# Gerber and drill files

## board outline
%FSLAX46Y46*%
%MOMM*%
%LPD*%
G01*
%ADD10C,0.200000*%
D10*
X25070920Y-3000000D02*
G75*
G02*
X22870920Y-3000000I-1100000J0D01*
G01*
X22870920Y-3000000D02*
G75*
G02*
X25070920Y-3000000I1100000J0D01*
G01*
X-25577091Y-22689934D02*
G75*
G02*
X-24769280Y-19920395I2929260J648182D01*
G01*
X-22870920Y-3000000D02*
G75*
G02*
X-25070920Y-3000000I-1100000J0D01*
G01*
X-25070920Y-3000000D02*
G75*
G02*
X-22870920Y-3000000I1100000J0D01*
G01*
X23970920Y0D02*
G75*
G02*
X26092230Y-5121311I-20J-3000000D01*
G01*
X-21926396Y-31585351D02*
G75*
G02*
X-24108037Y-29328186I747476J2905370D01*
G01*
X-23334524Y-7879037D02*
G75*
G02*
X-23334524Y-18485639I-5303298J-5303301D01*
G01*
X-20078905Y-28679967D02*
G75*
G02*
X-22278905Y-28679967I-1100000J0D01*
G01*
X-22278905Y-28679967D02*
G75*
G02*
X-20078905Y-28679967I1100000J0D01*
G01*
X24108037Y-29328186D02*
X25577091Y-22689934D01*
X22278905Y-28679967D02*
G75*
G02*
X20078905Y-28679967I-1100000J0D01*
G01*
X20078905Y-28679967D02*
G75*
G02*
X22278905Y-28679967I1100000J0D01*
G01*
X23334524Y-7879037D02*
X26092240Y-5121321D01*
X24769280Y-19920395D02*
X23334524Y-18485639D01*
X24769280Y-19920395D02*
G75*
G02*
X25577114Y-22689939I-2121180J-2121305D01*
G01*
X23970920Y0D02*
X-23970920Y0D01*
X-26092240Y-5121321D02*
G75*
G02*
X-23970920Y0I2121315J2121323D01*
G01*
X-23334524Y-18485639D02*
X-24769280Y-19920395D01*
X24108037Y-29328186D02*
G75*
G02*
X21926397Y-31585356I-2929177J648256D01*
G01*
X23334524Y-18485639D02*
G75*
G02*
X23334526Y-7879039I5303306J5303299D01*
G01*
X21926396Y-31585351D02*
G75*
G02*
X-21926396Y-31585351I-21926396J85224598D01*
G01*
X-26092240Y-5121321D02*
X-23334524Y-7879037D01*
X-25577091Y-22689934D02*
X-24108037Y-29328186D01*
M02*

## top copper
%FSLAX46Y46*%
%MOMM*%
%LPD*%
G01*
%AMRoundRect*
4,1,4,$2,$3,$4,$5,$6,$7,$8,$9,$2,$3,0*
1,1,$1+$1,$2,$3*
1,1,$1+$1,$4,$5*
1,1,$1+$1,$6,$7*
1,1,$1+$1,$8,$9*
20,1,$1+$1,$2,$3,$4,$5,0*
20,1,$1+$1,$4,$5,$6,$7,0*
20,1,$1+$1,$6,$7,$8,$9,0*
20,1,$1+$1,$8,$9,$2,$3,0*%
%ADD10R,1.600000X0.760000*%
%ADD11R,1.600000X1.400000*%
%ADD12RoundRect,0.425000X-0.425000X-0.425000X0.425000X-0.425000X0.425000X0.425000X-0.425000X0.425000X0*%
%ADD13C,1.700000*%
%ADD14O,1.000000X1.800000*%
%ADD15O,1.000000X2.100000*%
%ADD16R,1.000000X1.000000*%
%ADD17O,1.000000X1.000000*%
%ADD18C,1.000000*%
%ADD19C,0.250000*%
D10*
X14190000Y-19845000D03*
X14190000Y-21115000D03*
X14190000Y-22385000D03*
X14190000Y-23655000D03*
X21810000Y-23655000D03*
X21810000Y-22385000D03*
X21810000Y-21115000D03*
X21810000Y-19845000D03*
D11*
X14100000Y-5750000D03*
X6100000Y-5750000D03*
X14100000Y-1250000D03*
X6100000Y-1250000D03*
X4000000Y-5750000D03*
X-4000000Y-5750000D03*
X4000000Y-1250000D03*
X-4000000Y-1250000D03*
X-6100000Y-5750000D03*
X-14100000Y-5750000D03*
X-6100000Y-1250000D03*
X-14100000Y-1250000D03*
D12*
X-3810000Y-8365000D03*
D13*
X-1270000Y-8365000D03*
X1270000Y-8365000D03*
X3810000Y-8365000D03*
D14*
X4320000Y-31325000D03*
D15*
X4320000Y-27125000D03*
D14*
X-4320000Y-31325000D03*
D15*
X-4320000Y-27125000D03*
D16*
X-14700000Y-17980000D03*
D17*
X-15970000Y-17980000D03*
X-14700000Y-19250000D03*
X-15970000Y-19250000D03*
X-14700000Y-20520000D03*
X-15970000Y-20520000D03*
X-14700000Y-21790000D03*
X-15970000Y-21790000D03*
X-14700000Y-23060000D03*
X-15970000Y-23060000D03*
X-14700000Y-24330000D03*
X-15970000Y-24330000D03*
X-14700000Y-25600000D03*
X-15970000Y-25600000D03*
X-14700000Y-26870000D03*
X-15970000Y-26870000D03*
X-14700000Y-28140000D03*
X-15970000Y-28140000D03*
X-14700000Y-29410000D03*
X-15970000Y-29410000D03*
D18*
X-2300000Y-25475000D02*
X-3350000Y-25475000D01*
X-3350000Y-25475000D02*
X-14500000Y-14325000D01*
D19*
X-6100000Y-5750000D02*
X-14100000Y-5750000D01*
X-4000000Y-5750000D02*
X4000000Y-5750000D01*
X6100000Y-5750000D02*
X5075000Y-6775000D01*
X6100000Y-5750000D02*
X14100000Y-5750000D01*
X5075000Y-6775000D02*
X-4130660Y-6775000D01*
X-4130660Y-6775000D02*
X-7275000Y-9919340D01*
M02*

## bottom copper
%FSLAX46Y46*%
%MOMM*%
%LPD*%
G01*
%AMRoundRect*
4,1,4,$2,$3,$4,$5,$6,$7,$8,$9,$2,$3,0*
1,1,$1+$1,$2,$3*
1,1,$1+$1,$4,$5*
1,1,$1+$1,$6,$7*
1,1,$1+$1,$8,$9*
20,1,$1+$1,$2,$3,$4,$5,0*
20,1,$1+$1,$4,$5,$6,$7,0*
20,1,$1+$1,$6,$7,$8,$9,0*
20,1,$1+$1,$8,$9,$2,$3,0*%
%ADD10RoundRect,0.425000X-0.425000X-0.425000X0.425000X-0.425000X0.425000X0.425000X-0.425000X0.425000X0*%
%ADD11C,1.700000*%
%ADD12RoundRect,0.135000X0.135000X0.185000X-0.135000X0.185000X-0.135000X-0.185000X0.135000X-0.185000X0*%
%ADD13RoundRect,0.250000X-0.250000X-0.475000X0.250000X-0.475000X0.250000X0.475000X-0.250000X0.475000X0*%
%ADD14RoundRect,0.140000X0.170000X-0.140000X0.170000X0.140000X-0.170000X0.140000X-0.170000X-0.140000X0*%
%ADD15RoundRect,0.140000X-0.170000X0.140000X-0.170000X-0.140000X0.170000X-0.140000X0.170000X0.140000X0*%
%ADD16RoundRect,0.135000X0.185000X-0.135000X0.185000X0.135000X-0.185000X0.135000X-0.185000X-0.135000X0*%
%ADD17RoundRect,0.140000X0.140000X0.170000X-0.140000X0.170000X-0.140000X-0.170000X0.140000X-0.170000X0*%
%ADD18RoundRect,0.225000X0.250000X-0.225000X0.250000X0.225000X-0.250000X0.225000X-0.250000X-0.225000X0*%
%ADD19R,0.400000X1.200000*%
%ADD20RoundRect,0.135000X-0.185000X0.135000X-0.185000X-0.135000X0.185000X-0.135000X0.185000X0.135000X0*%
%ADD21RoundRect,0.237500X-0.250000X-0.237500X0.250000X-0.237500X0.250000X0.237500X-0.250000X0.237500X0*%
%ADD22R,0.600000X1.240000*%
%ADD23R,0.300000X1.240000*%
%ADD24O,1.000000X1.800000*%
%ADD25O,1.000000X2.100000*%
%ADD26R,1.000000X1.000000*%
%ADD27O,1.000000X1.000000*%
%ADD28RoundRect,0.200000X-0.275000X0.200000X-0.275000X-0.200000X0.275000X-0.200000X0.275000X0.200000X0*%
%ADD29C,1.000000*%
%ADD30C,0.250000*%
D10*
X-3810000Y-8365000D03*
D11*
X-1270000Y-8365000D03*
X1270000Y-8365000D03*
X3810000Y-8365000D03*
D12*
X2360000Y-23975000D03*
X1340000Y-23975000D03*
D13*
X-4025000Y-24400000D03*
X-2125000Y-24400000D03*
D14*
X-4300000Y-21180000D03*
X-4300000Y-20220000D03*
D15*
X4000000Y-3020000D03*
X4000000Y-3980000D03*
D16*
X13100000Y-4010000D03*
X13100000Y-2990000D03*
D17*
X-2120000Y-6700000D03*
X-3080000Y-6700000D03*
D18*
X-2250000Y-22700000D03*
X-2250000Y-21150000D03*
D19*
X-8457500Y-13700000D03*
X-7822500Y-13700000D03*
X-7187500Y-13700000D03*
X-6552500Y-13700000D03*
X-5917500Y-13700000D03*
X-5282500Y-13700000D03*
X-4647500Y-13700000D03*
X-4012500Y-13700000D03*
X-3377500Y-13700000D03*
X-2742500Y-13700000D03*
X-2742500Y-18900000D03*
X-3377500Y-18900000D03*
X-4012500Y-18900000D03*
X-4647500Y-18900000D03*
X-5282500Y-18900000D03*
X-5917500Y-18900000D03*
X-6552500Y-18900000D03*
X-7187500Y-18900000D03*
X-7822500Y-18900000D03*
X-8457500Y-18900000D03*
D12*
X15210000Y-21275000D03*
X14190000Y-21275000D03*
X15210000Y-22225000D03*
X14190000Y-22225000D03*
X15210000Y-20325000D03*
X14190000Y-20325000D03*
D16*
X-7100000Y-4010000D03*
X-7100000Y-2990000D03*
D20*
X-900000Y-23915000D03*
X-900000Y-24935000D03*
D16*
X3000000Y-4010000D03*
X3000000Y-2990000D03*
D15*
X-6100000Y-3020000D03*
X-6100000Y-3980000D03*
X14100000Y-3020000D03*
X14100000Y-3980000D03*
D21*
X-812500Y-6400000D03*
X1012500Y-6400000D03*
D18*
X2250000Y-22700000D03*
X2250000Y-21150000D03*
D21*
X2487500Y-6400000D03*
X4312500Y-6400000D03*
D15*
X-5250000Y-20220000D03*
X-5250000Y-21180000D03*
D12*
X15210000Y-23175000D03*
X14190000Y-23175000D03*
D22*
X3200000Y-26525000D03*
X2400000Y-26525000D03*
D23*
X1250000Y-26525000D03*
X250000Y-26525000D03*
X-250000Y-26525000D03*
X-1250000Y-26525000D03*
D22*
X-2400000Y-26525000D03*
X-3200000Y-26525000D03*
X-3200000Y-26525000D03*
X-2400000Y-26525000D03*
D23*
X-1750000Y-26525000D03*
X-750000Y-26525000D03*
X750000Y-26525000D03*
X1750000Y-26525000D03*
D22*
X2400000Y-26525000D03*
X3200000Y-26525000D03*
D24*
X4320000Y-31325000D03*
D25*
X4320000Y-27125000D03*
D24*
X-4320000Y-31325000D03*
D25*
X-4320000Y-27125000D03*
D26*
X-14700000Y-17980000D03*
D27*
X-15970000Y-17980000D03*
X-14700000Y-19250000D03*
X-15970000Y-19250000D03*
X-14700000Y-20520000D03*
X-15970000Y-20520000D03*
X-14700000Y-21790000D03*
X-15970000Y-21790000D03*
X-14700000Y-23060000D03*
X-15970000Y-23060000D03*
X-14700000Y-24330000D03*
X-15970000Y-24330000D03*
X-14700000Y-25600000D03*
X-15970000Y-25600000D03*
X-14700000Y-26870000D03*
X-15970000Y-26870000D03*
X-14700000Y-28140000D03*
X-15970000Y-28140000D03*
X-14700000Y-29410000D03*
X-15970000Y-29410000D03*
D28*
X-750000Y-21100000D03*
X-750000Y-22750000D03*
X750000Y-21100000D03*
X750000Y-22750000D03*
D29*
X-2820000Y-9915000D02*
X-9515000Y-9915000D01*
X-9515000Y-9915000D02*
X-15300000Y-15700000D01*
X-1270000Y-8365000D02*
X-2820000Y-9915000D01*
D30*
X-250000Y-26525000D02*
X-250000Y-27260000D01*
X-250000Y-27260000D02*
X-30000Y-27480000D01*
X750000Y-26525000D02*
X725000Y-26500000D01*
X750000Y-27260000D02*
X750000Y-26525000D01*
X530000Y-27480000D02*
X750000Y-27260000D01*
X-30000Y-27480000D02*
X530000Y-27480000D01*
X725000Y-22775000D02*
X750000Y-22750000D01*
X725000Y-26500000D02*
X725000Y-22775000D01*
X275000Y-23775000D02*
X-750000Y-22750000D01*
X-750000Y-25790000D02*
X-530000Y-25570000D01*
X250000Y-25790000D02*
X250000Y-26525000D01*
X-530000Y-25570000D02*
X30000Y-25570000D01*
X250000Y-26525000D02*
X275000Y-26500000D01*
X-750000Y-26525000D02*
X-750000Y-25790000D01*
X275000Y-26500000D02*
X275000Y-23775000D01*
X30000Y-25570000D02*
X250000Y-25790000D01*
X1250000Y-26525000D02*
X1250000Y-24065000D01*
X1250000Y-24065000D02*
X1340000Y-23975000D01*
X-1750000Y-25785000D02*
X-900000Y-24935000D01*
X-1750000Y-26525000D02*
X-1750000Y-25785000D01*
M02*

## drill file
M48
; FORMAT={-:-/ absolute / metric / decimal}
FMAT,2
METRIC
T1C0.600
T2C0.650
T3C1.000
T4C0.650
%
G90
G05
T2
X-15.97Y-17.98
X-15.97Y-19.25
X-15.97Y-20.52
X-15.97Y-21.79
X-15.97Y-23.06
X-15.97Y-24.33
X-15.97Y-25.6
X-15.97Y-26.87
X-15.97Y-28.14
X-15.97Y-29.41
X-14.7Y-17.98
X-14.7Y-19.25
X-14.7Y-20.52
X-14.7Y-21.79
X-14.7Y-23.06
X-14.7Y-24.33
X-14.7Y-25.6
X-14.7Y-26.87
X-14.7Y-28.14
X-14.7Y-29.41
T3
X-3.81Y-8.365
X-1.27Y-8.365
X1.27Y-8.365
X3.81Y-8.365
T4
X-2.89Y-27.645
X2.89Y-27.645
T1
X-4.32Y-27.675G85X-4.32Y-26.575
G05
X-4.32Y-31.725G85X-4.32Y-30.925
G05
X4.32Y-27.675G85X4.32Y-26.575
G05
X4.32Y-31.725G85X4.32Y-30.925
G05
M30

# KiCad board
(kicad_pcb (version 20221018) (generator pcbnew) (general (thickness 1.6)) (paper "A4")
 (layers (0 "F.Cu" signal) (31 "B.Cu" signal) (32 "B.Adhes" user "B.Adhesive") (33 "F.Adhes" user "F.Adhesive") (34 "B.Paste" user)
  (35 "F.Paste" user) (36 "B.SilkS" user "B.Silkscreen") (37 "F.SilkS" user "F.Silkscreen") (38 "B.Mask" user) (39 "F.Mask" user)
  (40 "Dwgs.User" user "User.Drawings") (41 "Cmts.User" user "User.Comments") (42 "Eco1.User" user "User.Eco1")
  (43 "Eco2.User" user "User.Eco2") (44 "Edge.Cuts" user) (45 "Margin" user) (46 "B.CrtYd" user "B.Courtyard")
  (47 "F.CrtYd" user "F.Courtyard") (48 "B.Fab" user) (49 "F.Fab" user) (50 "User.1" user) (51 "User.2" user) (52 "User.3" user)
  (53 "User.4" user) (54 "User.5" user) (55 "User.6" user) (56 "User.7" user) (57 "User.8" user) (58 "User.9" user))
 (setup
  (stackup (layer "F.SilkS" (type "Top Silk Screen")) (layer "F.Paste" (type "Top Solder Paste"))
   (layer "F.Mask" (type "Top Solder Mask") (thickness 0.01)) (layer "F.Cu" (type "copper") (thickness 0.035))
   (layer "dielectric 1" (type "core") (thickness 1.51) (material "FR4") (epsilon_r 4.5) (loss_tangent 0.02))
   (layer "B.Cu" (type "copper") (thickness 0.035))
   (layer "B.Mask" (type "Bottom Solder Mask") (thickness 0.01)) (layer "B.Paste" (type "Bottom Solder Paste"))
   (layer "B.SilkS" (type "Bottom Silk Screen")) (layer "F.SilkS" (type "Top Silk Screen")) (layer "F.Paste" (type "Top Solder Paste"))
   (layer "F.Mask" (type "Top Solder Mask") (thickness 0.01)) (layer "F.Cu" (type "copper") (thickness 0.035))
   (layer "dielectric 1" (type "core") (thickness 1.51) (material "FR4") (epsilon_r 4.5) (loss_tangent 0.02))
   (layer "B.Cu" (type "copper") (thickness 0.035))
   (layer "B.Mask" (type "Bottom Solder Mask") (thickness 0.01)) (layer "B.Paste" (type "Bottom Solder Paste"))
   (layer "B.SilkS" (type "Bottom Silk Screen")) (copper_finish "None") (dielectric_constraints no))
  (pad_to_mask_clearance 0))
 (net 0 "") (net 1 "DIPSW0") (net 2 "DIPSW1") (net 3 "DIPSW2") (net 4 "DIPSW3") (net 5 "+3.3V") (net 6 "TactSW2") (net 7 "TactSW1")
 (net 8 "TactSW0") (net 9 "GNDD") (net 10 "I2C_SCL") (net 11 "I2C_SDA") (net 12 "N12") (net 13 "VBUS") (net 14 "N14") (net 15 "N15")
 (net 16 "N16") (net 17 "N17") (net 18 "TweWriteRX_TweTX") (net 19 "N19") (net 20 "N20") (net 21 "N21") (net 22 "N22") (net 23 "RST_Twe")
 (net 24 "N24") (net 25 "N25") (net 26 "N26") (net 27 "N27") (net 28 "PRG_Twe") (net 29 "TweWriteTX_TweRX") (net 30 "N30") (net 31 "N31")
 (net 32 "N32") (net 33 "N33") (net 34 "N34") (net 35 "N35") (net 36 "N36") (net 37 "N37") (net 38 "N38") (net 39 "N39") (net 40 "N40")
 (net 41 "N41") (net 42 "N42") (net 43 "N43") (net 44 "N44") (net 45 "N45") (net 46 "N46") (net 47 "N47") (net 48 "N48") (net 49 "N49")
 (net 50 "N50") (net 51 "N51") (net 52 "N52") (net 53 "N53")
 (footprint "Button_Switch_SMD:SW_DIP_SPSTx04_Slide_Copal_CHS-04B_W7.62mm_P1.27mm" (layer "F.Cu") (at 18 21.75)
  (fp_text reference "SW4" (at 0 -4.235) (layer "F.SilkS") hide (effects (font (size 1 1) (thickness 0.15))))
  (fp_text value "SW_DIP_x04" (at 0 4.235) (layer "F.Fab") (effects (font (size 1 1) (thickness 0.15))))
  (pad "1" smd rect (at -3.81 -1.905) (size 1.6 0.76) (layers "F.Cu" "F.Paste" "F.Mask") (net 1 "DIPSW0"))
  (pad "2" smd rect (at -3.81 -0.635) (size 1.6 0.76) (layers "F.Cu" "F.Paste" "F.Mask") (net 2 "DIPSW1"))
  (pad "3" smd rect (at -3.81 0.635) (size 1.6 0.76) (layers "F.Cu" "F.Paste" "F.Mask") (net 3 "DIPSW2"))
  (pad "4" smd rect (at -3.81 1.905) (size 1.6 0.76) (layers "F.Cu" "F.Paste" "F.Mask") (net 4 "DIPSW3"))
  (pad "5" smd rect (at 3.81 1.905) (size 1.6 0.76) (layers "F.Cu" "F.Paste" "F.Mask") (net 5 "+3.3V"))
  (pad "6" smd rect (at 3.81 0.635) (size 1.6 0.76) (layers "F.Cu" "F.Paste" "F.Mask") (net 5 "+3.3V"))
  (pad "7" smd rect (at 3.81 -0.635) (size 1.6 0.76) (layers "F.Cu" "F.Paste" "F.Mask") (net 5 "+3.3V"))
  (pad "8" smd rect (at 3.81 -1.905) (size 1.6 0.76) (layers "F.Cu" "F.Paste" "F.Mask") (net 5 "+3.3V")))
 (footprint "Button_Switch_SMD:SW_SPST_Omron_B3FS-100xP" (layer "F.Cu") (at 10.1 3.5 180)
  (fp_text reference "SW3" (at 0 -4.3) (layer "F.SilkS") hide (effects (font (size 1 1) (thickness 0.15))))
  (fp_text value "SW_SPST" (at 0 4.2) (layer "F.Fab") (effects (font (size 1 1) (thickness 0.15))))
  (pad "1" smd rect (at -4 -2.25) (size 1.6 1.4) (layers "F.Cu" "F.Paste" "F.Mask") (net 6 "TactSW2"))
  (pad "1" smd rect (at 4 -2.25) (size 1.6 1.4) (layers "F.Cu" "F.Paste" "F.Mask") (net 6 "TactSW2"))
  (pad "2" smd rect (at -4 2.25) (size 1.6 1.4) (layers "F.Cu" "F.Paste" "F.Mask") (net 5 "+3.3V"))
  (pad "2" smd rect (at 4 2.25) (size 1.6 1.4) (layers "F.Cu" "F.Paste" "F.Mask") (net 5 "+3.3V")))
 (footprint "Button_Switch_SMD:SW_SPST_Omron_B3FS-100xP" (layer "F.Cu") (at 0 3.5 180)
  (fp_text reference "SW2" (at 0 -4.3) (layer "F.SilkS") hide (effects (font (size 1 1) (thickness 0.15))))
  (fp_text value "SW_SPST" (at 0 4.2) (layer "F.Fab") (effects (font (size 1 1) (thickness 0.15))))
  (pad "1" smd rect (at -4 -2.25) (size 1.6 1.4) (layers "F.Cu" "F.Paste" "F.Mask") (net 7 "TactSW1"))
  (pad "1" smd rect (at 4 -2.25) (size 1.6 1.4) (layers "F.Cu" "F.Paste" "F.Mask") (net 7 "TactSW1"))
  (pad "2" smd rect (at -4 2.25) (size 1.6 1.4) (layers "F.Cu" "F.Paste" "F.Mask") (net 5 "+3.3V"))
  (pad "2" smd rect (at 4 2.25) (size 1.6 1.4) (layers "F.Cu" "F.Paste" "F.Mask") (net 5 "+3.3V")))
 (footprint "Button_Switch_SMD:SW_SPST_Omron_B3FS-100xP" (layer "F.Cu") (at -10.1 3.5 180)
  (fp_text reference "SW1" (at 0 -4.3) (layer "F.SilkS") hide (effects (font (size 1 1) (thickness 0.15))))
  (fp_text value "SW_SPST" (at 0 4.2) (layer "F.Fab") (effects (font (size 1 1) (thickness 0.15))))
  (pad "1" smd rect (at -4 -2.25) (size 1.6 1.4) (layers "F.Cu" "F.Paste" "F.Mask") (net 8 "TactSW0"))
  (pad "1" smd rect (at 4 -2.25) (size 1.6 1.4) (layers "F.Cu" "F.Paste" "F.Mask") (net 8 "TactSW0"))
  (pad "2" smd rect (at -4 2.25) (size 1.6 1.4) (layers "F.Cu" "F.Paste" "F.Mask") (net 5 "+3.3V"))
  (pad "2" smd rect (at 4 2.25) (size 1.6 1.4) (layers "F.Cu" "F.Paste" "F.Mask") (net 5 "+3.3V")))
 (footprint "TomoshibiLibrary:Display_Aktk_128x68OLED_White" (layer "F.Cu") (at 0 7.095)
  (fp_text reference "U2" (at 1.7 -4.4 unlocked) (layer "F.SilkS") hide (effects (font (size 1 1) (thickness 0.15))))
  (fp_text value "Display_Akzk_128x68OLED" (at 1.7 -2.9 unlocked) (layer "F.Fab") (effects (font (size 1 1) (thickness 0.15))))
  (pad "1" thru_hole roundrect (at -3.81 1.27) (size 1.7 1.7) (drill 1) (layers "*.Cu" "*.Mask") (roundrect_rratio 0.25) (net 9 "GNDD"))
  (pad "2" thru_hole circle (at -1.27 1.27) (size 1.7 1.7) (drill 1) (layers "*.Cu" "*.Mask") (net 5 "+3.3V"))
  (pad "3" thru_hole circle (at 1.27 1.27) (size 1.7 1.7) (drill 1) (layers "*.Cu" "*.Mask") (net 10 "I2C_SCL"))
  (pad "4" thru_hole circle (at 3.81 1.27) (size 1.7 1.7) (drill 1) (layers "*.Cu" "*.Mask") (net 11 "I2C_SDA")))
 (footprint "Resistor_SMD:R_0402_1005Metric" (layer "B.Cu") (at 1.85 23.975 180)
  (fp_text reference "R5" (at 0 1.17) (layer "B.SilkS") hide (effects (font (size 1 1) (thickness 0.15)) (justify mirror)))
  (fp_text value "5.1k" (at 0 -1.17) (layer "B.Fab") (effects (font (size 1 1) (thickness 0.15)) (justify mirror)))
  (pad "1" smd roundrect (at -0.51 0 180) (size 0.54 0.64) (layers "B.Cu" "B.Paste" "B.Mask") (roundrect_rratio 0.25) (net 9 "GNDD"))
  (pad "2" smd roundrect (at 0.51 0 180) (size 0.54 0.64) (layers "B.Cu" "B.Paste" "B.Mask") (roundrect_rratio 0.25) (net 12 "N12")))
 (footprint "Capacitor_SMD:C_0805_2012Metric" (layer "B.Cu") (at -3.075 24.4)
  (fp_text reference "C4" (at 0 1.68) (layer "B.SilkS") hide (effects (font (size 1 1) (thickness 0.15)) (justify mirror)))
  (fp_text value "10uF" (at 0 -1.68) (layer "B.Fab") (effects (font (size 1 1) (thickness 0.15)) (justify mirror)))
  (pad "1" smd roundrect (at -0.95 0) (size 1 1.45) (layers "B.Cu" "B.Paste" "B.Mask") (roundrect_rratio 0.25) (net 9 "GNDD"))
  (pad "2" smd roundrect (at 0.95 0) (size 1 1.45) (layers "B.Cu" "B.Paste" "B.Mask") (roundrect_rratio 0.25) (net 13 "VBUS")))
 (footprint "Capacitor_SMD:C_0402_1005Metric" (layer "B.Cu") (at -4.3 20.7 90)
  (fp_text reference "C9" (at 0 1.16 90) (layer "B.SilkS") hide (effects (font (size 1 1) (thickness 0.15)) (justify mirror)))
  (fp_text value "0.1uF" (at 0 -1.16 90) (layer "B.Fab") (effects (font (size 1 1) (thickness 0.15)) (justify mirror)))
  (pad "1" smd roundrect (at -0.48 0 90) (size 0.56 0.62) (layers "B.Cu" "B.Paste" "B.Mask") (roundrect_rratio 0.25) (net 9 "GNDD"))
  (pad "2" smd roundrect (at 0.48 0 90) (size 0.56 0.62) (layers "B.Cu" "B.Paste" "B.Mask") (roundrect_rratio 0.25) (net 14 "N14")))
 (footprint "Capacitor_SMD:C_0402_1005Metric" (layer "B.Cu") (at 4 3.5 -90)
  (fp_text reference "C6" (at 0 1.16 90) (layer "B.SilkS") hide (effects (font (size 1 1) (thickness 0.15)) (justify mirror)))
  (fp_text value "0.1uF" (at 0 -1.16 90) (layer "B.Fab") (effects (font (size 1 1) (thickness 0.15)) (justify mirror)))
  (pad "1" smd roundrect (at -0.48 0 270) (size 0.56 0.62) (layers "B.Cu" "B.Paste" "B.Mask") (roundrect_rratio 0.25) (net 5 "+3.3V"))
  (pad "2" smd roundrect (at 0.48 0 270) (size 0.56 0.62) (layers "B.Cu" "B.Paste" "B.Mask") (roundrect_rratio 0.25) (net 7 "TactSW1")))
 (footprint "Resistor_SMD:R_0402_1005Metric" (layer "B.Cu") (at 13.1 3.5 90)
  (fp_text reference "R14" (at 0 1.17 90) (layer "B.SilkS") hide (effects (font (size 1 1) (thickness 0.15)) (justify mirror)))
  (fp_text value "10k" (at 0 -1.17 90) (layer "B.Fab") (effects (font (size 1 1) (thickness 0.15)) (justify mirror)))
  (pad "1" smd roundrect (at -0.51 0 90) (size 0.54 0.64) (layers "B.Cu" "B.Paste" "B.Mask") (roundrect_rratio 0.25) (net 6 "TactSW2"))
  (pad "2" smd roundrect (at 0.51 0 90) (size 0.54 0.64) (layers "B.Cu" "B.Paste" "B.Mask") (roundrect_rratio 0.25) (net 9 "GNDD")))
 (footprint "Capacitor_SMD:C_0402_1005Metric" (layer "B.Cu") (at -2.6 6.7 180)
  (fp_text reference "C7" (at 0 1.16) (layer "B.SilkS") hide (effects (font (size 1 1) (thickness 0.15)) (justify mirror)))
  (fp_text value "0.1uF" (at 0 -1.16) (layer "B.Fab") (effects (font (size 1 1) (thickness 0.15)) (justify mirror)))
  (pad "1" smd roundrect (at -0.48 0 180) (size 0.56 0.62) (layers "B.Cu" "B.Paste" "B.Mask") (roundrect_rratio 0.25) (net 5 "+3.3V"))
  (pad "2" smd roundrect (at 0.48 0 180) (size 0.56 0.62) (layers "B.Cu" "B.Paste" "B.Mask") (roundrect_rratio 0.25) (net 9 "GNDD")))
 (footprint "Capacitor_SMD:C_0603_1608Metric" (layer "B.Cu") (at -2.25 21.925 90)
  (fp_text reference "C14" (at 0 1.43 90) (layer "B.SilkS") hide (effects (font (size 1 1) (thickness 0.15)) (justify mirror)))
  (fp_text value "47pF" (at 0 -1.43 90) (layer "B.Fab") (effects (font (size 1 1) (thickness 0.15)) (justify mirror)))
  (pad "1" smd roundrect (at -0.775 0 90) (size 0.9 0.95) (layers "B.Cu" "B.Paste" "B.Mask") (roundrect_rratio 0.25) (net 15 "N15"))
  (pad "2" smd roundrect (at 0.775 0 90) (size 0.9 0.95) (layers "B.Cu" "B.Paste" "B.Mask") (roundrect_rratio 0.25) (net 9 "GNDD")))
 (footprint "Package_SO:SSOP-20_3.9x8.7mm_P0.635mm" (layer "B.Cu") (at -5.6 16.3 -90)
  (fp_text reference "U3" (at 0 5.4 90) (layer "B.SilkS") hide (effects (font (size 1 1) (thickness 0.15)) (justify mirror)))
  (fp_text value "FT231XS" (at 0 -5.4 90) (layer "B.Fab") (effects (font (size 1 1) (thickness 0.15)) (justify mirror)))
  (pad "1" smd rect (at -2.6 2.8575 270) (size 1.2 0.4) (layers "B.Cu" "B.Paste" "B.Mask") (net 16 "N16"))
  (pad "2" smd rect (at -2.6 2.2225 270) (size 1.2 0.4) (layers "B.Cu" "B.Paste" "B.Mask") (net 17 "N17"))
  (pad "3" smd rect (at -2.6 1.5875 270) (size 1.2 0.4) (layers "B.Cu" "B.Paste" "B.Mask") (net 14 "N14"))
  (pad "4" smd rect (at -2.6 0.9525 270) (size 1.2 0.4) (layers "B.Cu" "B.Paste" "B.Mask") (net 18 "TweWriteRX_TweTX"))
  (pad "5" smd rect (at -2.6 0.3175 270) (size 1.2 0.4) (layers "B.Cu" "B.Paste" "B.Mask") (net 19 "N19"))
  (pad "6" smd rect (at -2.6 -0.3175 270) (size 1.2 0.4) (layers "B.Cu" "B.Paste" "B.Mask") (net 9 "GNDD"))
  (pad "7" smd rect (at -2.6 -0.9525 270) (size 1.2 0.4) (layers "B.Cu" "B.Paste" "B.Mask") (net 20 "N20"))
  (pad "8" smd rect (at -2.6 -1.5875 270) (size 1.2 0.4) (layers "B.Cu" "B.Paste" "B.Mask") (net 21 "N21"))
  (pad "9" smd rect (at -2.6 -2.2225 270) (size 1.2 0.4) (layers "B.Cu" "B.Paste" "B.Mask") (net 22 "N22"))
  (pad "10" smd rect (at -2.6 -2.8575 270) (size 1.2 0.4) (layers "B.Cu" "B.Paste" "B.Mask") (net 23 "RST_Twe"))
  (pad "11" smd rect (at 2.6 -2.8575 270) (size 1.2 0.4) (layers "B.Cu" "B.Paste" "B.Mask") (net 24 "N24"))
  (pad "12" smd rect (at 2.6 -2.2225 270) (size 1.2 0.4) (layers "B.Cu" "B.Paste" "B.Mask") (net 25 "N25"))
  (pad "13" smd rect (at 2.6 -1.5875 270) (size 1.2 0.4) (layers "B.Cu" "B.Paste" "B.Mask") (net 14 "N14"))
  (pad "14" smd rect (at 2.6 -0.9525 270) (size 1.2 0.4) (layers "B.Cu" "B.Paste" "B.Mask") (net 14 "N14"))
  (pad "15" smd rect (at 2.6 -0.3175 270) (size 1.2 0.4) (layers "B.Cu" "B.Paste" "B.Mask") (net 13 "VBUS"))
  (pad "16" smd rect (at 2.6 0.3175 270) (size 1.2 0.4) (layers "B.Cu" "B.Paste" "B.Mask") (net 9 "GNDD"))
  (pad "17" smd rect (at 2.6 0.9525 270) (size 1.2 0.4) (layers "B.Cu" "B.Paste" "B.Mask") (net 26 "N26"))
  (pad "18" smd rect (at 2.6 1.5875 270) (size 1.2 0.4) (layers "B.Cu" "B.Paste" "B.Mask") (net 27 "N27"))
  (pad "19" smd rect (at 2.6 2.2225 270) (size 1.2 0.4) (layers "B.Cu" "B.Paste" "B.Mask") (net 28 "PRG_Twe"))
  (pad "20" smd rect (at 2.6 2.8575 270) (size 1.2 0.4) (layers "B.Cu" "B.Paste" "B.Mask") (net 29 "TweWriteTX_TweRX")))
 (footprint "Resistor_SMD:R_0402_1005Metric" (layer "B.Cu") (at 14.7 21.275 180)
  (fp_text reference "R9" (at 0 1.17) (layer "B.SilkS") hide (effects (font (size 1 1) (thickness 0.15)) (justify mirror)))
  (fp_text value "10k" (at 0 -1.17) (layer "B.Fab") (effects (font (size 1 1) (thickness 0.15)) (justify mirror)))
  (pad "1" smd roundrect (at -0.51 0 180) (size 0.54 0.64) (layers "B.Cu" "B.Paste" "B.Mask") (roundrect_rratio 0.25) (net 9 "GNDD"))
  (pad "2" smd roundrect (at 0.51 0 180) (size 0.54 0.64) (layers "B.Cu" "B.Paste" "B.Mask") (roundrect_rratio 0.25) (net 2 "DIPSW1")))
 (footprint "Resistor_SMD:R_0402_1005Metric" (layer "B.Cu") (at 14.7 22.225 180)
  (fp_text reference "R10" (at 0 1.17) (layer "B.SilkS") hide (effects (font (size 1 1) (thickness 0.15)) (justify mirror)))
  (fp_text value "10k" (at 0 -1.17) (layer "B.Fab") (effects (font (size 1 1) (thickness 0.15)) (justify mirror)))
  (pad "1" smd roundrect (at -0.51 0 180) (size 0.54 0.64) (layers "B.Cu" "B.Paste" "B.Mask") (roundrect_rratio 0.25) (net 9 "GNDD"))
  (pad "2" smd roundrect (at 0.51 0 180) (size 0.54 0.64) (layers "B.Cu" "B.Paste" "B.Mask") (roundrect_rratio 0.25) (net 3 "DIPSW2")))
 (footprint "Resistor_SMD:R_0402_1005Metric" (layer "B.Cu") (at 14.7 20.325 180)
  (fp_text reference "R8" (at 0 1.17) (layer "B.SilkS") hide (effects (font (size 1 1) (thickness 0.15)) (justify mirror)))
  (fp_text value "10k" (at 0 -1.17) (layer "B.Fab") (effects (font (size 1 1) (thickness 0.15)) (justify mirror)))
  (pad "1" smd roundrect (at -0.51 0 180) (size 0.54 0.64) (layers "B.Cu" "B.Paste" "B.Mask") (roundrect_rratio 0.25) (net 9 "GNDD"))
  (pad "2" smd roundrect (at 0.51 0 180) (size 0.54 0.64) (layers "B.Cu" "B.Paste" "B.Mask") (roundrect_rratio 0.25) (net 1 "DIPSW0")))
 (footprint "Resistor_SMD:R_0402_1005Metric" (layer "B.Cu") (at -7.1 3.5 90)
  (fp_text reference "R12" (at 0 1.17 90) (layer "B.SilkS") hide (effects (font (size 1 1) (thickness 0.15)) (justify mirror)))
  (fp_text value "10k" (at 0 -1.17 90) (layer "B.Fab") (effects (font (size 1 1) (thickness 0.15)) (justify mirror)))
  (pad "1" smd roundrect (at -0.51 0 90) (size 0.54 0.64) (layers "B.Cu" "B.Paste" "B.Mask") (roundrect_rratio 0.25) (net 8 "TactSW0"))
  (pad "2" smd roundrect (at 0.51 0 90) (size 0.54 0.64) (layers "B.Cu" "B.Paste" "B.Mask") (roundrect_rratio 0.25) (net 9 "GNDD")))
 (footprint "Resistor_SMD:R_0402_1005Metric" (layer "B.Cu") (at -0.9 24.425 -90)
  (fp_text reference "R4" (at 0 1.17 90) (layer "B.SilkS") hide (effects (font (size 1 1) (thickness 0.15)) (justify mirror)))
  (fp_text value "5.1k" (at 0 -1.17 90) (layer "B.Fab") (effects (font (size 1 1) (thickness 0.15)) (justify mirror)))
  (pad "1" smd roundrect (at -0.51 0 270) (size 0.54 0.64) (layers "B.Cu" "B.Paste" "B.Mask") (roundrect_rratio 0.25) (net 9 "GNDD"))
  (pad "2" smd roundrect (at 0.51 0 270) (size 0.54 0.64) (layers "B.Cu" "B.Paste" "B.Mask") (roundrect_rratio 0.25) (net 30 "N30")))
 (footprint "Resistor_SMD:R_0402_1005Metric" (layer "B.Cu") (at 3 3.5 90)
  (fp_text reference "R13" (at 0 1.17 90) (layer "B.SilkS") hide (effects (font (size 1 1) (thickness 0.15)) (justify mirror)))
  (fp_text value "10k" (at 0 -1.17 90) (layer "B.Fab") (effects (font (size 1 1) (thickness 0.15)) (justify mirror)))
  (pad "1" smd roundrect (at -0.51 0 90) (size 0.54 0.64) (layers "B.Cu" "B.Paste" "B.Mask") (roundrect_rratio 0.25) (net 7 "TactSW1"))
  (pad "2" smd roundrect (at 0.51 0 90) (size 0.54 0.64) (layers "B.Cu" "B.Paste" "B.Mask") (roundrect_rratio 0.25) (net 9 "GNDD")))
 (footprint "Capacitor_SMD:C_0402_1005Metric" (layer "B.Cu") (at -6.1 3.5 -90)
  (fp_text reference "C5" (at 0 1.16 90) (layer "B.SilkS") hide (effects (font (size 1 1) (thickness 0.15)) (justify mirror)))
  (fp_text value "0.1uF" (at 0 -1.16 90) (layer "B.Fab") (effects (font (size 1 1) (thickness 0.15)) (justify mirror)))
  (pad "1" smd roundrect (at -0.48 0 270) (size 0.56 0.62) (layers "B.Cu" "B.Paste" "B.Mask") (roundrect_rratio 0.25) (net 5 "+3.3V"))
  (pad "2" smd roundrect (at 0.48 0 270) (size 0.56 0.62) (layers "B.Cu" "B.Paste" "B.Mask") (roundrect_rratio 0.25) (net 8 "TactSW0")))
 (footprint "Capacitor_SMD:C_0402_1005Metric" (layer "B.Cu") (at 14.1 3.5 -90)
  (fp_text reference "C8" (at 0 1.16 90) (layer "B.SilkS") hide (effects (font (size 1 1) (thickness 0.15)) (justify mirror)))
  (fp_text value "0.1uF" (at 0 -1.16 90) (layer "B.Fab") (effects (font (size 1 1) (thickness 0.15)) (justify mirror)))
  (pad "1" smd roundrect (at -0.48 0 270) (size 0.56 0.62) (layers "B.Cu" "B.Paste" "B.Mask") (roundrect_rratio 0.25) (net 5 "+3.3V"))
  (pad "2" smd roundrect (at 0.48 0 270) (size 0.56 0.62) (layers "B.Cu" "B.Paste" "B.Mask") (roundrect_rratio 0.25) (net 6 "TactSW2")))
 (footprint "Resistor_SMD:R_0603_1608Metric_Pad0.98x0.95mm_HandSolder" (layer "B.Cu") (at 0.1 6.4)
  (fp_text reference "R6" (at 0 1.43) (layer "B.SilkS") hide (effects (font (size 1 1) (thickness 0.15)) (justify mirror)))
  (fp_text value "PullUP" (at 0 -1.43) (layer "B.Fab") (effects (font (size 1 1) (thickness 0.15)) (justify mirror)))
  (pad "1" smd roundrect (at -0.9125 0) (size 0.975 0.95) (layers "B.Cu" "B.Paste" "B.Mask") (roundrect_rratio 0.25) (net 5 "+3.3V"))
  (pad "2" smd roundrect (at 0.9125 0) (size 0.975 0.95) (layers "B.Cu" "B.Paste" "B.Mask") (roundrect_rratio 0.25) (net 10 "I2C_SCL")))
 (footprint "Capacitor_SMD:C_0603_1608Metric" (layer "B.Cu") (at 2.25 21.925 90)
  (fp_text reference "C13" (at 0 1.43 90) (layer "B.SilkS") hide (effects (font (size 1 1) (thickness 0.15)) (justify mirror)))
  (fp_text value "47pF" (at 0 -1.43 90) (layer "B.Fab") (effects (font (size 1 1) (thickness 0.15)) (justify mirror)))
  (pad "1" smd roundrect (at -0.775 0 90) (size 0.9 0.95) (layers "B.Cu" "B.Paste" "B.Mask") (roundrect_rratio 0.25) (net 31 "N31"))
  (pad "2" smd roundrect (at 0.775 0 90) (size 0.9 0.95) (layers "B.Cu" "B.Paste" "B.Mask") (roundrect_rratio 0.25) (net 9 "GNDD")))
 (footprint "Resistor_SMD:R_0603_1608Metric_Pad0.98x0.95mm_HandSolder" (layer "B.Cu") (at 3.4 6.4)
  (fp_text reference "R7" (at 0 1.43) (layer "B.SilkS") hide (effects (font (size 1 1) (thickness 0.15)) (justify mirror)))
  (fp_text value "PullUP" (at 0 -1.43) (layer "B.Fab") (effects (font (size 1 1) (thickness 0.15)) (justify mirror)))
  (pad "1" smd roundrect (at -0.9125 0) (size 0.975 0.95) (layers "B.Cu" "B.Paste" "B.Mask") (roundrect_rratio 0.25) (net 5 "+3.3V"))
  (pad "2" smd roundrect (at 0.9125 0) (size 0.975 0.95) (layers "B.Cu" "B.Paste" "B.Mask") (roundrect_rratio 0.25) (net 11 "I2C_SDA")))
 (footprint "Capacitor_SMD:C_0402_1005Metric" (layer "B.Cu") (at -5.25 20.7 -90)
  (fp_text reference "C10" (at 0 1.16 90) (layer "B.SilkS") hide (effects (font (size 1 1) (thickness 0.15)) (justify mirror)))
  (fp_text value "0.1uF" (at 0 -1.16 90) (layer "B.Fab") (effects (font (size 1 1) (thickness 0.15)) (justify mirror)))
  (pad "1" smd roundrect (at -0.48 0 270) (size 0.56 0.62) (layers "B.Cu" "B.Paste" "B.Mask") (roundrect_rratio 0.25) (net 13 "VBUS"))
  (pad "2" smd roundrect (at 0.48 0 270) (size 0.56 0.62) (layers "B.Cu" "B.Paste" "B.Mask") (roundrect_rratio 0.25) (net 9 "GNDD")))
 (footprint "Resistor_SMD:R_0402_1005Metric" (layer "B.Cu") (at 14.7 23.175 180)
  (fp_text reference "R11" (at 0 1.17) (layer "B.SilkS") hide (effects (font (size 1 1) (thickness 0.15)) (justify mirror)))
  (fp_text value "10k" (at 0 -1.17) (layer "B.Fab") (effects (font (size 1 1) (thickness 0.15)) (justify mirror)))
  (pad "1" smd roundrect (at -0.51 0 180) (size 0.54 0.64) (layers "B.Cu" "B.Paste" "B.Mask") (roundrect_rratio 0.25) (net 9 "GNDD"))
  (pad "2" smd roundrect (at 0.51 0 180) (size 0.54 0.64) (layers "B.Cu" "B.Paste" "B.Mask") (roundrect_rratio 0.25) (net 4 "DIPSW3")))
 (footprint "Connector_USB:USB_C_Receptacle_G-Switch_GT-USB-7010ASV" (layer "B.Cu") (at 0 30.25 180)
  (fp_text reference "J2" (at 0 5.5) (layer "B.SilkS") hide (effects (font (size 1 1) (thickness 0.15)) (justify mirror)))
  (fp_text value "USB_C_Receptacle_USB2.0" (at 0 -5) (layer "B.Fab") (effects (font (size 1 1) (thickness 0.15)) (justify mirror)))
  (pad "" np_thru_hole circle (at -2.89 2.605 180) (size 0.65 0.65) (drill 0.65) (layers "*.Cu" "*.Mask"))
  (pad "" np_thru_hole circle (at 2.89 2.605 180) (size 0.65 0.65) (drill 0.65) (layers "*.Cu" "*.Mask"))
  (pad "A1" smd rect (at -3.2 3.725 180) (size 0.6 1.24) (layers "B.Cu" "B.Paste" "B.Mask") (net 9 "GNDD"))
  (pad "A4" smd rect (at -2.4 3.725 180) (size 0.6 1.24) (layers "B.Cu" "B.Paste" "B.Mask") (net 13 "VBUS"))
  (pad "A5" smd rect (at -1.25 3.725 180) (size 0.3 1.24) (layers "B.Cu" "B.Paste" "B.Mask") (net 12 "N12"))
  (pad "A6" smd rect (at -0.25 3.725 180) (size 0.3 1.24) (layers "B.Cu" "B.Paste" "B.Mask") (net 15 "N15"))
  (pad "A7" smd rect (at 0.25 3.725 180) (size 0.3 1.24) (layers "B.Cu" "B.Paste" "B.Mask") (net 31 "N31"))
  (pad "A8" smd rect (at 1.25 3.725 180) (size 0.3 1.24) (layers "B.Cu" "B.Paste" "B.Mask") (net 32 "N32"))
  (pad "A9" smd rect (at 2.4 3.725 180) (size 0.6 1.24) (layers "B.Cu" "B.Paste" "B.Mask") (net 13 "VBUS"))
  (pad "A12" smd rect (at 3.2 3.725 180) (size 0.6 1.24) (layers "B.Cu" "B.Paste" "B.Mask") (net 9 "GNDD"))
  (pad "B1" smd rect (at 3.2 3.725 180) (size 0.6 1.24) (layers "B.Cu" "B.Paste" "B.Mask") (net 9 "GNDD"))
  (pad "B4" smd rect (at 2.4 3.725 180) (size 0.6 1.24) (layers "B.Cu" "B.Paste" "B.Mask") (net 13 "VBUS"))
  (pad "B5" smd rect (at 1.75 3.725 180) (size 0.3 1.24) (layers "B.Cu" "B.Paste" "B.Mask") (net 30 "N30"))
  (pad "B6" smd rect (at 0.75 3.725 180) (size 0.3 1.24) (layers "B.Cu" "B.Paste" "B.Mask") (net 15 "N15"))
  (pad "B7" smd rect (at -0.75 3.725 180) (size 0.3 1.24) (layers "B.Cu" "B.Paste" "B.Mask") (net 31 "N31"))
  (pad "B8" smd rect (at -1.75 3.725 180) (size 0.3 1.24) (layers "B.Cu" "B.Paste" "B.Mask") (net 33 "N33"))
  (pad "B9" smd rect (at -2.4 3.725 180) (size 0.6 1.24) (layers "B.Cu" "B.Paste" "B.Mask") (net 13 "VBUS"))
  (pad "B12" smd rect (at -3.2 3.725 180) (size 0.6 1.24) (layers "B.Cu" "B.Paste" "B.Mask") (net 9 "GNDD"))
  (pad "S1" thru_hole oval (at -4.32 -1.075 180) (size 1 1.8) (drill oval 0.6 1.4) (layers "*.Cu" "*.Mask") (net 9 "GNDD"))
  (pad "S1" thru_hole oval (at -4.32 3.125 180) (size 1 2.1) (drill oval 0.6 1.7) (layers "*.Cu" "*.Mask") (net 9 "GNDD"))
  (pad "S1" thru_hole oval (at 4.32 -1.075 180) (size 1 1.8) (drill oval 0.6 1.4) (layers "*.Cu" "*.Mask") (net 9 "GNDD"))
  (pad "S1" thru_hole oval (at 4.32 3.125 180) (size 1 2.1) (drill oval 0.6 1.7) (layers "*.Cu" "*.Mask") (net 9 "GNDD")))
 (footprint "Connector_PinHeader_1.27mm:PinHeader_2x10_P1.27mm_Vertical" (layer "B.Cu") (at -14.7 17.98 180)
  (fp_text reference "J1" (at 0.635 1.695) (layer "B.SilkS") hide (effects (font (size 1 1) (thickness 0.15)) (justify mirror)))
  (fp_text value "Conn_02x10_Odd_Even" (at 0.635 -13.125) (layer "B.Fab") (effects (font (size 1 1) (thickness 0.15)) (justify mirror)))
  (pad "1" thru_hole rect (at 0 0 180) (size 1 1) (drill 0.65) (layers "*.Cu" "*.Mask") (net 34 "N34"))
  (pad "2" thru_hole oval (at 1.27 0 180) (size 1 1) (drill 0.65) (layers "*.Cu" "*.Mask") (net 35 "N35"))
  (pad "3" thru_hole oval (at 0 -1.27 180) (size 1 1) (drill 0.65) (layers "*.Cu" "*.Mask") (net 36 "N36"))
  (pad "4" thru_hole oval (at 1.27 -1.27 180) (size 1 1) (drill 0.65) (layers "*.Cu" "*.Mask") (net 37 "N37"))
  (pad "5" thru_hole oval (at 0 -2.54 180) (size 1 1) (drill 0.65) (layers "*.Cu" "*.Mask") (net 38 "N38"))
  (pad "6" thru_hole oval (at 1.27 -2.54 180) (size 1 1) (drill 0.65) (layers "*.Cu" "*.Mask") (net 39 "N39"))
  (pad "7" thru_hole oval (at 0 -3.81 180) (size 1 1) (drill 0.65) (layers "*.Cu" "*.Mask") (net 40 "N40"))
  (pad "8" thru_hole oval (at 1.27 -3.81 180) (size 1 1) (drill 0.65) (layers "*.Cu" "*.Mask") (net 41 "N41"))
  (pad "9" thru_hole oval (at 0 -5.08 180) (size 1 1) (drill 0.65) (layers "*.Cu" "*.Mask") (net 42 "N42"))
  (pad "10" thru_hole oval (at 1.27 -5.08 180) (size 1 1) (drill 0.65) (layers "*.Cu" "*.Mask") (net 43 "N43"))
  (pad "11" thru_hole oval (at 0 -6.35 180) (size 1 1) (drill 0.65) (layers "*.Cu" "*.Mask") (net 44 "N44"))
  (pad "12" thru_hole oval (at 1.27 -6.35 180) (size 1 1) (drill 0.65) (layers "*.Cu" "*.Mask") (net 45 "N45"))
  (pad "13" thru_hole oval (at 0 -7.62 180) (size 1 1) (drill 0.65) (layers "*.Cu" "*.Mask") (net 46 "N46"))
  (pad "14" thru_hole oval (at 1.27 -7.62 180) (size 1 1) (drill 0.65) (layers "*.Cu" "*.Mask") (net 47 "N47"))
  (pad "15" thru_hole oval (at 0 -8.89 180) (size 1 1) (drill 0.65) (layers "*.Cu" "*.Mask") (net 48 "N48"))
  (pad "16" thru_hole oval (at 1.27 -8.89 180) (size 1 1) (drill 0.65) (layers "*.Cu" "*.Mask") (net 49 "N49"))
  (pad "17" thru_hole oval (at 0 -10.16 180) (size 1 1) (drill 0.65) (layers "*.Cu" "*.Mask") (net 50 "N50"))
  (pad "18" thru_hole oval (at 1.27 -10.16 180) (size 1 1) (drill 0.65) (layers "*.Cu" "*.Mask") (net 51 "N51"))
  (pad "19" thru_hole oval (at 0 -11.43 180) (size 1 1) (drill 0.65) (layers "*.Cu" "*.Mask") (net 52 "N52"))
  (pad "20" thru_hole oval (at 1.27 -11.43 180) (size 1 1) (drill 0.65) (layers "*.Cu" "*.Mask") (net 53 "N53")))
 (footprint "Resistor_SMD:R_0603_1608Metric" (layer "B.Cu") (at -0.75 21.925 -90)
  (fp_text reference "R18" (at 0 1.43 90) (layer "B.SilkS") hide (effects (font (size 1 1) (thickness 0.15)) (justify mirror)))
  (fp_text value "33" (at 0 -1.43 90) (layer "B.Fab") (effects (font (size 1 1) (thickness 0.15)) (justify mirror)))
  (pad "1" smd roundrect (at -0.825 0 270) (size 0.8 0.95) (layers "B.Cu" "B.Paste" "B.Mask") (roundrect_rratio 0.25) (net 24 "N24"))
  (pad "2" smd roundrect (at 0.825 0 270) (size 0.8 0.95) (layers "B.Cu" "B.Paste" "B.Mask") (roundrect_rratio 0.25) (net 15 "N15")))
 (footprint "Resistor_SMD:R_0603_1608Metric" (layer "B.Cu") (at 0.75 21.925 -90)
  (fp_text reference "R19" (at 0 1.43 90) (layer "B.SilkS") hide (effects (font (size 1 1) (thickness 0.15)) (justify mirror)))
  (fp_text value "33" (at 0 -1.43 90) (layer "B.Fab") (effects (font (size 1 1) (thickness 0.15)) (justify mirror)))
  (pad "1" smd roundrect (at -0.825 0 270) (size 0.8 0.95) (layers "B.Cu" "B.Paste" "B.Mask") (roundrect_rratio 0.25) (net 25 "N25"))
  (pad "2" smd roundrect (at 0.825 0 270) (size 0.8 0.95) (layers "B.Cu" "B.Paste" "B.Mask") (roundrect_rratio 0.25) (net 31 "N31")))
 (gr_circle (center 23.97092 3) (end 23.97092 4.1) (stroke (width 0.2) (type solid)) (fill none) (layer "Edge.Cuts"))
 (gr_arc (start -25.577091 22.689934) (mid -25.527937 21.201697) (end -24.76928 19.920395) (stroke (width 0.2) (type solid))
  (layer "Edge.Cuts"))
 (gr_circle (center -23.97092 3) (end -23.97092 4.1) (stroke (width 0.2) (type solid)) (fill none) (layer "Edge.Cuts"))
 (gr_arc (start 23.97092 0) (mid 26.742556 1.851949) (end 26.09224 5.121321) (stroke (width 0.2) (type solid)) (layer "Edge.Cuts"))
 (gr_arc (start -21.926396 31.585351) (mid -23.33601 30.764893) (end -24.108037 29.328186) (stroke (width 0.2) (type solid))
  (layer "Edge.Cuts"))
 (gr_arc (start -23.334524 7.879037) (mid -21.137824 13.182338) (end -23.334524 18.485639) (stroke (width 0.2) (type solid))
  (layer "Edge.Cuts"))
 (gr_circle (center -21.178905 28.679967) (end -21.178905 29.779967) (stroke (width 0.2) (type solid)) (fill none) (layer "Edge.Cuts"))
 (gr_line (start 24.108037 29.328186) (end 25.577091 22.689934) (stroke (width 0.2) (type solid)) (layer "Edge.Cuts"))
 (gr_circle (center 21.178905 28.679967) (end 21.178905 29.779967) (stroke (width 0.2) (type solid)) (fill none) (layer "Edge.Cuts"))
 (gr_line (start 23.334524 7.879037) (end 26.09224 5.121321) (stroke (width 0.2) (type solid)) (layer "Edge.Cuts"))
 (gr_line (start 24.76928 19.920395) (end 23.334524 18.485639) (stroke (width 0.2) (type solid)) (layer "Edge.Cuts"))
 (gr_arc (start 24.76928 19.920395) (mid 25.527976 21.201686) (end 25.577091 22.689934) (stroke (width 0.2) (type solid))
  (layer "Edge.Cuts"))
 (gr_line (start 23.97092 0) (end -23.97092 0) (stroke (width 0.2) (type solid)) (layer "Edge.Cuts"))
 (gr_arc (start -26.09224 5.121321) (mid -26.742561 1.851947) (end -23.97092 0) (stroke (width 0.2) (type solid)) (layer "Edge.Cuts"))
 (gr_line (start -23.334524 18.485639) (end -24.76928 19.920395) (stroke (width 0.2) (type solid)) (layer "Edge.Cuts"))
 (gr_arc (start 24.108037 29.328186) (mid 23.336002 30.764885) (end 21.926396 31.585351) (stroke (width 0.2) (type solid))
  (layer "Edge.Cuts"))
 (gr_arc (start 23.334524 18.485639) (mid 21.137826 13.182338) (end 23.334524 7.879037) (stroke (width 0.2) (type solid))
  (layer "Edge.Cuts"))
 (gr_arc (start 21.926396 31.585351) (mid 0 34.360747) (end -21.926396 31.585351) (stroke (width 0.2) (type solid)) (layer "Edge.Cuts"))
 (gr_line (start -26.09224 5.121321) (end -23.334524 7.879037) (stroke (width 0.2) (type solid)) (layer "Edge.Cuts"))
 (gr_line (start -25.577091 22.689934) (end -24.108037 29.328186) (stroke (width 0.2) (type solid)) (layer "Edge.Cuts"))
 (segment (start -2.3 25.475) (end -3.35 25.475) (width 1) (layer "F.Cu") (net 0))
 (segment (start -3.35 25.475) (end -14.5 14.325) (width 1) (layer "F.Cu") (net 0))
 (segment (start -2.82 9.915) (end -9.515 9.915) (width 1) (layer "B.Cu") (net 5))
 (segment (start -9.515 9.915) (end -15.3 15.7) (width 1) (layer "B.Cu") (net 5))
 (segment (start -1.27 8.365) (end -2.82 9.915) (width 1) (layer "B.Cu") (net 5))
 (segment (start -6.1 5.75) (end -14.1 5.75) (width 0.25) (layer "F.Cu") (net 8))
 (segment (start -4 5.75) (end 4 5.75) (width 0.25) (layer "F.Cu") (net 7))
 (segment (start 6.1 5.75) (end 5.075 6.775) (width 0.25) (layer "F.Cu") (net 6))
 (segment (start 6.1 5.75) (end 14.1 5.75) (width 0.25) (layer "F.Cu") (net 6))
 (segment (start 5.075 6.775) (end -4.13066 6.775) (width 0.25) (layer "F.Cu") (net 6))
 (segment (start -4.13066 6.775) (end -7.275 9.91934) (width 0.25) (layer "F.Cu") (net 6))
 (segment (start -0.25 26.525) (end -0.25 27.26) (width 0.25) (layer "B.Cu") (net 31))
 (segment (start -0.25 27.26) (end -0.03 27.48) (width 0.25) (layer "B.Cu") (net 31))
 (segment (start 0.75 26.525) (end 0.725 26.5) (width 0.25) (layer "B.Cu") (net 31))
 (segment (start 0.75 27.26) (end 0.75 26.525) (width 0.25) (layer "B.Cu") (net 31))
 (segment (start 0.53 27.48) (end 0.75 27.26) (width 0.25) (layer "B.Cu") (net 31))
 (segment (start -0.03 27.48) (end 0.53 27.48) (width 0.25) (layer "B.Cu") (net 31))
 (segment (start 0.725 22.775) (end 0.75 22.75) (width 0.25) (layer "B.Cu") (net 31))
 (segment (start 0.725 26.5) (end 0.725 22.775) (width 0.25) (layer "B.Cu") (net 31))
 (segment (start 0.275 23.775) (end -0.75 22.75) (width 0.25) (layer "B.Cu") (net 15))
 (segment (start -0.75 25.79) (end -0.53 25.57) (width 0.25) (layer "B.Cu") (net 15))
 (segment (start 0.25 25.79) (end 0.25 26.525) (width 0.25) (layer "B.Cu") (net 15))
 (segment (start -0.53 25.57) (end 0.03 25.57) (width 0.25) (layer "B.Cu") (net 15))
 (segment (start 0.25 26.525) (end 0.275 26.5) (width 0.25) (layer "B.Cu") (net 15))
 (segment (start -0.75 26.525) (end -0.75 25.79) (width 0.25) (layer "B.Cu") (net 15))
 (segment (start 0.275 26.5) (end 0.275 23.775) (width 0.25) (layer "B.Cu") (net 15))
 (segment (start 0.03 25.57) (end 0.25 25.79) (width 0.25) (layer "B.Cu") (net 15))
 (segment (start 1.25 26.525) (end 1.25 24.065) (width 0.25) (layer "B.Cu") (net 12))
 (segment (start 1.25 24.065) (end 1.34 23.975) (width 0.25) (layer "B.Cu") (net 12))
 (segment (start -1.75 25.785) (end -0.9 24.935) (width 0.25) (layer "B.Cu") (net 30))
 (segment (start -1.75 26.525) (end -1.75 25.785) (width 0.25) (layer "B.Cu") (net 30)))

